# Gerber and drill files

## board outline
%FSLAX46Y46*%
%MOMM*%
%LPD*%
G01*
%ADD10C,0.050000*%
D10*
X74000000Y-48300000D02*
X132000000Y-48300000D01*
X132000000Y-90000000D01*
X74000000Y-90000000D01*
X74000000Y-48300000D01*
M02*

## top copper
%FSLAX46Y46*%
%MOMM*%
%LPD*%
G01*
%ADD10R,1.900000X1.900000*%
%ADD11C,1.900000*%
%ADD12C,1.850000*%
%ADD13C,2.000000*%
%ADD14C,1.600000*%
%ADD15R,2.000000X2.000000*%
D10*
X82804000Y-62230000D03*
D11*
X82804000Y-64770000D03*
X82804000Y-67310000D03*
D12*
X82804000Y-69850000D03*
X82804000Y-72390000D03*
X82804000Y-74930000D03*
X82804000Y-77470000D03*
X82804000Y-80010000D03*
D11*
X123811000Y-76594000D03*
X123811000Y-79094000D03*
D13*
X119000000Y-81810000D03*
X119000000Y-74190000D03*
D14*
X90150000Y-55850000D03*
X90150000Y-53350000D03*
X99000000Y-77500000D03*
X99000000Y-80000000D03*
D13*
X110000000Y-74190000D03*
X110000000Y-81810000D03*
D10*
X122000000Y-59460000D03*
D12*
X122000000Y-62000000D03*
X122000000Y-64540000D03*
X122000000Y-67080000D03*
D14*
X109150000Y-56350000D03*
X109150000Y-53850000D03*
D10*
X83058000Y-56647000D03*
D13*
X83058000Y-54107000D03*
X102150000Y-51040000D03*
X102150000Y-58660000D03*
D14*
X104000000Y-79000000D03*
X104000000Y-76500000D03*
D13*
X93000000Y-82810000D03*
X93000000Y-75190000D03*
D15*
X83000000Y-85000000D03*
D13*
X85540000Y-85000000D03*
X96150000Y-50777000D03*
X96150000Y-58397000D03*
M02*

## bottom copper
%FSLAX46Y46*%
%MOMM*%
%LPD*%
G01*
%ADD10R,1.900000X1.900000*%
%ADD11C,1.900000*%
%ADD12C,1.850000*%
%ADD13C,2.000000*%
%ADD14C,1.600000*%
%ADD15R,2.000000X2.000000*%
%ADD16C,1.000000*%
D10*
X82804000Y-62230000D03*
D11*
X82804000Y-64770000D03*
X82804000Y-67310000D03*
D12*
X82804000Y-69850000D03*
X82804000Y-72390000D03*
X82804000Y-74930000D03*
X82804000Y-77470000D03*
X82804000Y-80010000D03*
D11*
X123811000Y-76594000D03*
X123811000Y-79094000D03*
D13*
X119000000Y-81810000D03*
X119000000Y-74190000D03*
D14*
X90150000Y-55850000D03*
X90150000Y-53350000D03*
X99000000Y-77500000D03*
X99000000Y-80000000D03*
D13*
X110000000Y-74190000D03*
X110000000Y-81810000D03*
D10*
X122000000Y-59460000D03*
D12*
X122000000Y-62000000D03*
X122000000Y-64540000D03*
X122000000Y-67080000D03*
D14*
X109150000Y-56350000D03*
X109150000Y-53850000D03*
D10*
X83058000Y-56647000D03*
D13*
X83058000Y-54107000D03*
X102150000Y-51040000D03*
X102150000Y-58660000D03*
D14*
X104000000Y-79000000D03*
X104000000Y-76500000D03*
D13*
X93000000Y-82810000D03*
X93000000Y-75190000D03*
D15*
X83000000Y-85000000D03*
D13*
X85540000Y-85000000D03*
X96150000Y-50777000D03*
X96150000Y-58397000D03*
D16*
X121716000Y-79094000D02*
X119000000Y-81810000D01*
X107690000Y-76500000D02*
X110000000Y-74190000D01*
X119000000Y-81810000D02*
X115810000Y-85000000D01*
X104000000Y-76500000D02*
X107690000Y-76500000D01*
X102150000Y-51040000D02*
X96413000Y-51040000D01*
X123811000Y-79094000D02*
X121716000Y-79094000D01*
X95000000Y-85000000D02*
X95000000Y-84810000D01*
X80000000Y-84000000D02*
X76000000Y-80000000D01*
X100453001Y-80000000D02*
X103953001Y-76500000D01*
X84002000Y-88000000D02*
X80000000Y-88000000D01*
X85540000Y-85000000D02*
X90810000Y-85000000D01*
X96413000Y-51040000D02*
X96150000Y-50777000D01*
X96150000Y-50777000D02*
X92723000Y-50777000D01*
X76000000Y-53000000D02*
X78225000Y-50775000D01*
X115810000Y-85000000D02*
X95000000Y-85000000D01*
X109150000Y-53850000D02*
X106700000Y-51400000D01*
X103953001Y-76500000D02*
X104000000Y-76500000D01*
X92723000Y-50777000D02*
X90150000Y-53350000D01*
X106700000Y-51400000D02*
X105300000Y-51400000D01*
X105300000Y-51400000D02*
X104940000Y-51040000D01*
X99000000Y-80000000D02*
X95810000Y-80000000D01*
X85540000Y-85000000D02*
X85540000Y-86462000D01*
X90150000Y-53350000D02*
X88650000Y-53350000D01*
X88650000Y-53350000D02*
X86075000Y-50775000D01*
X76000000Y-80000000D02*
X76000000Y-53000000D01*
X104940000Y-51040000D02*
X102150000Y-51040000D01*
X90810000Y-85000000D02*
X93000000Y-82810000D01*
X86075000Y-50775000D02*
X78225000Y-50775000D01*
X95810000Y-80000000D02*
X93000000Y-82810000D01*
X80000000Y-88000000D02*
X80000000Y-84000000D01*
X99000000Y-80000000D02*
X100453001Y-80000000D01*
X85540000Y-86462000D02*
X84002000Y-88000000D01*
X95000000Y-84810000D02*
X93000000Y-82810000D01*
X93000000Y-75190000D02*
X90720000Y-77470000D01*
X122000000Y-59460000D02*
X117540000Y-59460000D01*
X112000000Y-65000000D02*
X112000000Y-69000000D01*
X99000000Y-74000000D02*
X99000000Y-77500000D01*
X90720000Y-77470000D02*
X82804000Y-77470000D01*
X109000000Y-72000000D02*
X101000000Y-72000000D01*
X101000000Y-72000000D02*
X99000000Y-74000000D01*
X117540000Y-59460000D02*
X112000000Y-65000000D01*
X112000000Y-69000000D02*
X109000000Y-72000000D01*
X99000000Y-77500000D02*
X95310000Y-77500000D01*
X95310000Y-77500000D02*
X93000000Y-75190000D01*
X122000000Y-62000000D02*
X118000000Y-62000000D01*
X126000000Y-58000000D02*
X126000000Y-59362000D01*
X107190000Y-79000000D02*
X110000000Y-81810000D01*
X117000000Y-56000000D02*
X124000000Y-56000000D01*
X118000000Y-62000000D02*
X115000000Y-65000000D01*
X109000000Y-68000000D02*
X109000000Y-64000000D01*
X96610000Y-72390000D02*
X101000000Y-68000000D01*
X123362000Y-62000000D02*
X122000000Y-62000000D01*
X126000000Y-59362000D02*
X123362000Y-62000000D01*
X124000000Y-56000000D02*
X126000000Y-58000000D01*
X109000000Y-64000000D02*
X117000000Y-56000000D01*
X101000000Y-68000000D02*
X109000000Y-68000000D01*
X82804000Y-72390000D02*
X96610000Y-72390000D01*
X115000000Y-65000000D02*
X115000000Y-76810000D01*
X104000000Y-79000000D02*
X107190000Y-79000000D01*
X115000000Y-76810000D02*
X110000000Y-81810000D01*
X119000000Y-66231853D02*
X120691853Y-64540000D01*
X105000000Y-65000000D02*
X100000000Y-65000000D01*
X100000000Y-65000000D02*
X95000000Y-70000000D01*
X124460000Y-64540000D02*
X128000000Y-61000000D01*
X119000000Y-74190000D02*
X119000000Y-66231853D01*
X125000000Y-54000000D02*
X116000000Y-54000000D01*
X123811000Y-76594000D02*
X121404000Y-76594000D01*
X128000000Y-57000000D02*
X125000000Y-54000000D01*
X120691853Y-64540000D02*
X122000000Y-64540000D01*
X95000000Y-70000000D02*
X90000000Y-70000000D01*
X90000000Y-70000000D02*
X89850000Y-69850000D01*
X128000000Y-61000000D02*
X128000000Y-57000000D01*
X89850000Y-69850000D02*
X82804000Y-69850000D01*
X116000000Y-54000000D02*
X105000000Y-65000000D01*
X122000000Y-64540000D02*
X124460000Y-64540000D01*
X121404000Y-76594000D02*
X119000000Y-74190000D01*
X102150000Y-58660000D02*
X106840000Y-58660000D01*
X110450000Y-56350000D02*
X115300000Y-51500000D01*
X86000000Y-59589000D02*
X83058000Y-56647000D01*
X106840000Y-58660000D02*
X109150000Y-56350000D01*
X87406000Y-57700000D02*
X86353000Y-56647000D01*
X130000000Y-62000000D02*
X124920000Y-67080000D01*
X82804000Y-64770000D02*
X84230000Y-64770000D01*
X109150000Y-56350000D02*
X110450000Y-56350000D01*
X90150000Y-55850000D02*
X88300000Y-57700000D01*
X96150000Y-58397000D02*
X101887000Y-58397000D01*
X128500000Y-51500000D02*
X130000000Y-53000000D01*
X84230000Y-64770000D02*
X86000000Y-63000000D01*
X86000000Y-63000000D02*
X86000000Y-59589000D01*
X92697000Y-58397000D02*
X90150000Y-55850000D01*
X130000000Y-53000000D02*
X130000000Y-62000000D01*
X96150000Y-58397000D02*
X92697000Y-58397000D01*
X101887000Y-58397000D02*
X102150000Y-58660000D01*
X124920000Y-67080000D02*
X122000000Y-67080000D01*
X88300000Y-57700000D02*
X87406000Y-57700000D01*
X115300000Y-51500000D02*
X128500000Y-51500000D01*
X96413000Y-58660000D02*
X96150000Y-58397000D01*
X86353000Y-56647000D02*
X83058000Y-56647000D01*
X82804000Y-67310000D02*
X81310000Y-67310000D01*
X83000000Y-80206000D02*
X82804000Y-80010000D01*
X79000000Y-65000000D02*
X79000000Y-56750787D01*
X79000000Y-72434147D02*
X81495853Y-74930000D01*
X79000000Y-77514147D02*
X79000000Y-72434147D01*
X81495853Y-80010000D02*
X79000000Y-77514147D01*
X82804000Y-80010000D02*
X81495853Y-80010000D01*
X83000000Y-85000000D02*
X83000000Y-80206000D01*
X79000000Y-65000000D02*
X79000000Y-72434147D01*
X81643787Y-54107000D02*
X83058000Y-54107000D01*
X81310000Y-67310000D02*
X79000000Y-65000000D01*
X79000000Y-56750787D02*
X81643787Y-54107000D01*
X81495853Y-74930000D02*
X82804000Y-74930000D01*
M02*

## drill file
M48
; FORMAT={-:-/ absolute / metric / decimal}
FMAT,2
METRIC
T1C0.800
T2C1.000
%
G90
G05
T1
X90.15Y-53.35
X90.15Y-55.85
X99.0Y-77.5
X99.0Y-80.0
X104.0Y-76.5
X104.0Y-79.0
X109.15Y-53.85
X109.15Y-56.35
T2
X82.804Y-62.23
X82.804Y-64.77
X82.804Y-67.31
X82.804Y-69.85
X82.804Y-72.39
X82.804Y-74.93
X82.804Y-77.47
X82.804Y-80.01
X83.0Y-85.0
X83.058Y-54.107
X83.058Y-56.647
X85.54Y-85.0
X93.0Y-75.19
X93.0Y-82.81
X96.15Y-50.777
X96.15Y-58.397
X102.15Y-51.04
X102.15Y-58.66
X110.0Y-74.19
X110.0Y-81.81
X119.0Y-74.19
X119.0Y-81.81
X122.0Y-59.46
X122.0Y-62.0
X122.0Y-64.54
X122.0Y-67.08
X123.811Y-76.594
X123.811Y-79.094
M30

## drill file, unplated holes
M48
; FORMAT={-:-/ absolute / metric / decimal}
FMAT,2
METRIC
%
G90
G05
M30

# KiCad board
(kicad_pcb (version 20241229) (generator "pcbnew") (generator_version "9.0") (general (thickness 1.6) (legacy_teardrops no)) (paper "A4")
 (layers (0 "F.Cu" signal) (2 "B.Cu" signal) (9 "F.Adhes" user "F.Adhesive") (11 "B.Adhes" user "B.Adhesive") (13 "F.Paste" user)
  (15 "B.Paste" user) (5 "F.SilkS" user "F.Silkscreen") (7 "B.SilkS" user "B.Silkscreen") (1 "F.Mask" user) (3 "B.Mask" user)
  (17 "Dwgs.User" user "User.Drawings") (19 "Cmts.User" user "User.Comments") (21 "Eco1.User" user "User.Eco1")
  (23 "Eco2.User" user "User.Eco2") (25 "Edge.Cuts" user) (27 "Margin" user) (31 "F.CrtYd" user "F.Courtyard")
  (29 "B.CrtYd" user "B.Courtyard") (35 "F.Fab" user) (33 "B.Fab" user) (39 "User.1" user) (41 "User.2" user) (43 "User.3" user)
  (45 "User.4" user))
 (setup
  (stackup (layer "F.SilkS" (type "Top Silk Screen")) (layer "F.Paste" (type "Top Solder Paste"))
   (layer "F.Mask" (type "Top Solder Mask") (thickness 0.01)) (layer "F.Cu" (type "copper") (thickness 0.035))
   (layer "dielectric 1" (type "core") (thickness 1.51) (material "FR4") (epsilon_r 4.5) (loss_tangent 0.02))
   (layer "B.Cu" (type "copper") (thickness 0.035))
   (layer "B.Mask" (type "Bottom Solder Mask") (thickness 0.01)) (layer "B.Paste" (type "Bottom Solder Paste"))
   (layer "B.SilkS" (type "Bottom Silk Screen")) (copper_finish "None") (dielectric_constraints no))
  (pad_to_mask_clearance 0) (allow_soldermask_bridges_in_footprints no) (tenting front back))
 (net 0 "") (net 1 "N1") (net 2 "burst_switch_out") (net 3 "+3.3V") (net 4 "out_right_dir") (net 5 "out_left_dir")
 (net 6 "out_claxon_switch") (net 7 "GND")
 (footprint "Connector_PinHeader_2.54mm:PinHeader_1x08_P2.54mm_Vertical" (layer "F.Cu") (at 82.804 62.23)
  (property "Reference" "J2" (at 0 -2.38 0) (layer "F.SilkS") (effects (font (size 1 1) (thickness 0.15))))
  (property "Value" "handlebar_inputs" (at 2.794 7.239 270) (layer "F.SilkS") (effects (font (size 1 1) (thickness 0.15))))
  (pad "1" thru_hole rect (at 0 0) (size 1.9 1.9) (drill 1) (layers "*.Cu" "*.Mask") (remove_unused_layers no) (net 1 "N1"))
  (pad "2" thru_hole circle (at 0 2.54) (size 1.9 1.9) (drill 1) (layers "*.Cu" "*.Mask") (remove_unused_layers no)
   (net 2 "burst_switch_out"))
  (pad "3" thru_hole circle (at 0 5.08) (size 1.9 1.9) (drill 1) (layers "*.Cu" "*.Mask") (remove_unused_layers no) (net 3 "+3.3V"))
  (pad "4" thru_hole circle (at 0 7.62) (size 1.85 1.85) (drill 1) (layers "*.Cu" "*.Mask") (remove_unused_layers no)
   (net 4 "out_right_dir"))
  (pad "5" thru_hole circle (at 0 10.16) (size 1.85 1.85) (drill 1) (layers "*.Cu" "*.Mask") (remove_unused_layers no)
   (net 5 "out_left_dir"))
  (pad "6" thru_hole circle (at 0 12.7) (size 1.85 1.85) (drill 1) (layers "*.Cu" "*.Mask") (remove_unused_layers no) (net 3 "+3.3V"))
  (pad "7" thru_hole circle (at 0 15.24) (size 1.85 1.85) (drill 1) (layers "*.Cu" "*.Mask") (remove_unused_layers no)
   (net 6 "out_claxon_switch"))
  (pad "8" thru_hole circle (at 0 17.78) (size 1.85 1.85) (drill 1) (layers "*.Cu" "*.Mask") (remove_unused_layers no) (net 3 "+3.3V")))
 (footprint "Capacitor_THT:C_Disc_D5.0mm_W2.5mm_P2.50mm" (layer "F.Cu") (at 123.811 76.594 -90)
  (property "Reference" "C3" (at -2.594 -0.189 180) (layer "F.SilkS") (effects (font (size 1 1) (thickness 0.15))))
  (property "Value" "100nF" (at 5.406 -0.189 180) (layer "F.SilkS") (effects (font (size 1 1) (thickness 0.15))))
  (pad "1" thru_hole circle (at 0 0 270) (size 1.9 1.9) (drill 1) (layers "*.Cu" "*.Mask") (remove_unused_layers no) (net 4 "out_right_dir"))
  (pad "2" thru_hole circle (at 2.5 0 270) (size 1.9 1.9) (drill 1) (layers "*.Cu" "*.Mask") (remove_unused_layers no) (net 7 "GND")))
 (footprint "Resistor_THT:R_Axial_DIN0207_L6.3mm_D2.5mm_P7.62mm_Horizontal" (layer "F.Cu") (at 119 81.81 90)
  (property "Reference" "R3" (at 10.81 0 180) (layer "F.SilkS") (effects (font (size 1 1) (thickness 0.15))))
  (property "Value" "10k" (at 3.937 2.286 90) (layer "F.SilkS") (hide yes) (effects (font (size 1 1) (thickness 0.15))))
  (pad "1" thru_hole circle (at 0 0 90) (size 2 2) (drill 1) (layers "*.Cu" "*.Mask") (remove_unused_layers no) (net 7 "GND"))
  (pad "2" thru_hole circle (at 7.62 0 90) (size 2 2) (drill 1) (layers "*.Cu" "*.Mask") (remove_unused_layers no) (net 4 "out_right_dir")))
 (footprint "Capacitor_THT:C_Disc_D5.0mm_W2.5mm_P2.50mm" (layer "F.Cu") (at 90.15 55.85 90)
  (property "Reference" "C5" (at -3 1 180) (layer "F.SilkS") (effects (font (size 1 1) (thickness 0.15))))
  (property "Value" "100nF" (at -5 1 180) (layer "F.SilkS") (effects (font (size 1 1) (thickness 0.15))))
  (pad "1" thru_hole circle (at 0 0 90) (size 1.6 1.6) (drill 0.8) (layers "*.Cu" "*.Mask") (remove_unused_layers no)
   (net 2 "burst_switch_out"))
  (pad "2" thru_hole circle (at 2.5 0 90) (size 1.6 1.6) (drill 0.8) (layers "*.Cu" "*.Mask") (remove_unused_layers no) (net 7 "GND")))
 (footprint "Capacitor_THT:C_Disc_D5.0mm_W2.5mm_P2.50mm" (layer "F.Cu") (at 99 77.5 -90)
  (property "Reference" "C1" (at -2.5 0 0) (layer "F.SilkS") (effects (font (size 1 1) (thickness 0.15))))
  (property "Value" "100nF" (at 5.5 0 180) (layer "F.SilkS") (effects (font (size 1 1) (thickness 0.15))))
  (pad "1" thru_hole circle (at 0 0 270) (size 1.6 1.6) (drill 0.8) (layers "*.Cu" "*.Mask") (remove_unused_layers no)
   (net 6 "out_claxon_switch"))
  (pad "2" thru_hole circle (at 2.5 0 270) (size 1.6 1.6) (drill 0.8) (layers "*.Cu" "*.Mask") (remove_unused_layers no) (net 7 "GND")))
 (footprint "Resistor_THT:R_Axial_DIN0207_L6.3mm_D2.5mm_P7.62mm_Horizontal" (layer "F.Cu") (at 110 74.19 -90)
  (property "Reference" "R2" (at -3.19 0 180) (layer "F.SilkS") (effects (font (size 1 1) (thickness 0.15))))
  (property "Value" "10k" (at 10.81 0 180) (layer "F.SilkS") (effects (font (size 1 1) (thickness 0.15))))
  (pad "1" thru_hole circle (at 0 0 270) (size 2 2) (drill 1) (layers "*.Cu" "*.Mask") (remove_unused_layers no) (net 7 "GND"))
  (pad "2" thru_hole circle (at 7.62 0 270) (size 2 2) (drill 1) (layers "*.Cu" "*.Mask") (remove_unused_layers no) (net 5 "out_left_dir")))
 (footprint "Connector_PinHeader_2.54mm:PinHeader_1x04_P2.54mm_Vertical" (layer "F.Cu") (at 122 59.46)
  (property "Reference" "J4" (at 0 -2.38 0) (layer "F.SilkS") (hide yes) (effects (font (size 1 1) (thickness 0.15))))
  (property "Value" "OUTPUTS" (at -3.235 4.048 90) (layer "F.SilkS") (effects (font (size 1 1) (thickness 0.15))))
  (pad "1" thru_hole rect (at 0 0) (size 1.9 1.9) (drill 1) (layers "*.Cu" "*.Mask") (remove_unused_layers no) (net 6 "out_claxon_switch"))
  (pad "2" thru_hole circle (at 0 2.54) (size 1.85 1.85) (drill 1) (layers "*.Cu" "*.Mask") (remove_unused_layers no) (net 5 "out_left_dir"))
  (pad "3" thru_hole circle (at 0 5.08) (size 1.85 1.85) (drill 1) (layers "*.Cu" "*.Mask") (remove_unused_layers no)
   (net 4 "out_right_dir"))
  (pad "4" thru_hole circle (at 0 7.62) (size 1.85 1.85) (drill 1) (layers "*.Cu" "*.Mask") (remove_unused_layers no)
   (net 2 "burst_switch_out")))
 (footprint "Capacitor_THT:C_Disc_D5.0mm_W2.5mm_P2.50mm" (layer "F.Cu") (at 109.15 56.35 90)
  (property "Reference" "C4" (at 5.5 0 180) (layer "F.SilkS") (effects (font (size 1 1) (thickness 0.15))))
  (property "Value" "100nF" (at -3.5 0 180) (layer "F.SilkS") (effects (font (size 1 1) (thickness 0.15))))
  (pad "1" thru_hole circle (at 0 0 90) (size 1.6 1.6) (drill 0.8) (layers "*.Cu" "*.Mask") (remove_unused_layers no)
   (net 2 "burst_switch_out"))
  (pad "2" thru_hole circle (at 2.5 0 90.798) (size 1.6 1.6) (drill 0.8) (layers "*.Cu" "*.Mask") (remove_unused_layers no) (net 7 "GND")))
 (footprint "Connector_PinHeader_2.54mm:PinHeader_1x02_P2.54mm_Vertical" (layer "F.Cu") (at 83.058 56.647 180)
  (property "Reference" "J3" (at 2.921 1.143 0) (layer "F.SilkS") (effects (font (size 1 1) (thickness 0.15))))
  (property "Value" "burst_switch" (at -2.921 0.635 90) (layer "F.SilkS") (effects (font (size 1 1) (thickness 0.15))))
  (pad "1" thru_hole rect (at 0 0 180) (size 1.9 1.9) (drill 1) (layers "*.Cu" "*.Mask") (remove_unused_layers no)
   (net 2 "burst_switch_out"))
  (pad "2" thru_hole circle (at 0 2.54 180) (size 2 2) (drill 1) (layers "*.Cu" "*.Mask") (remove_unused_layers no) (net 3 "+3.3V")))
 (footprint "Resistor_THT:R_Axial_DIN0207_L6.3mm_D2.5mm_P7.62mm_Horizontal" (layer "F.Cu") (at 102.15 51.04 -90)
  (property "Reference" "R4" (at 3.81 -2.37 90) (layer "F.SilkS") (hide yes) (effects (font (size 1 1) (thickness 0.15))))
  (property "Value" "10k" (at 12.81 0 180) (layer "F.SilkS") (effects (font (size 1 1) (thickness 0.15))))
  (pad "1" thru_hole circle (at 0 0 270) (size 2 2) (drill 1) (layers "*.Cu" "*.Mask") (remove_unused_layers no) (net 7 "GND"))
  (pad "2" thru_hole circle (at 7.62 0 270) (size 2 2) (drill 1) (layers "*.Cu" "*.Mask") (remove_unused_layers no)
   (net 2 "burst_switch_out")))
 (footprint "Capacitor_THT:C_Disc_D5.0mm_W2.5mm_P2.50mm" (layer "F.Cu") (at 104 79 90)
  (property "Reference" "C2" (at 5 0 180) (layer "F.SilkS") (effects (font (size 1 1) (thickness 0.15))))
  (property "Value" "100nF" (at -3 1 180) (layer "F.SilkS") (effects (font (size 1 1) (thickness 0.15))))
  (pad "1" thru_hole circle (at 0 0 90) (size 1.6 1.6) (drill 0.8) (layers "*.Cu" "*.Mask") (remove_unused_layers no) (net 5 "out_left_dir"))
  (pad "2" thru_hole circle (at 2.5 0 90) (size 1.6 1.6) (drill 0.8) (layers "*.Cu" "*.Mask") (remove_unused_layers no) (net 7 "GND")))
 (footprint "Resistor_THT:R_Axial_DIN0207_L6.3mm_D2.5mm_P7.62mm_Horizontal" (layer "F.Cu") (at 93 82.81 90)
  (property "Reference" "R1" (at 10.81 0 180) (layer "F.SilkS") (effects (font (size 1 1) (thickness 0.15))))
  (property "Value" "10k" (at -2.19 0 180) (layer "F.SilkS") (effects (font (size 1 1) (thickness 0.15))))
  (pad "1" thru_hole circle (at 0 0 90) (size 2 2) (drill 1) (layers "*.Cu" "*.Mask") (remove_unused_layers no) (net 7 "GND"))
  (pad "2" thru_hole circle (at 7.62 0 90) (size 2 2) (drill 1) (layers "*.Cu" "*.Mask") (remove_unused_layers no)
   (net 6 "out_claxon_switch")))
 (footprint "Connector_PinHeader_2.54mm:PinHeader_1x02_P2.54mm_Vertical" (layer "F.Cu") (at 83 85 90)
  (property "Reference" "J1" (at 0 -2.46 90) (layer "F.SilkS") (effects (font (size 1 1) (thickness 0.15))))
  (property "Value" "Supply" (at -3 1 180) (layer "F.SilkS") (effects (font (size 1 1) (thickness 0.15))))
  (pad "1" thru_hole rect (at 0 0 90) (size 2 2) (drill 1) (layers "*.Cu" "*.Mask") (remove_unused_layers no) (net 3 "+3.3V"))
  (pad "2" thru_hole circle (at 0 2.54 90) (size 2 2) (drill 1) (layers "*.Cu" "*.Mask") (remove_unused_layers no) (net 7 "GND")))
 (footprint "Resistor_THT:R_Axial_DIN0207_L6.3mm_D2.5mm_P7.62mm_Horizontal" (layer "F.Cu") (at 96.15 50.777 -90)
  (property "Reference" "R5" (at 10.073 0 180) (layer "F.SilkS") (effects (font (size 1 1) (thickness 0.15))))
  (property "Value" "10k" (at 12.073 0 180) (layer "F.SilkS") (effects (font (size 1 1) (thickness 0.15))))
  (pad "1" thru_hole circle (at 0 0 270) (size 2 2) (drill 1) (layers "*.Cu" "*.Mask") (remove_unused_layers no) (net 7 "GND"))
  (pad "2" thru_hole circle (at 7.62 0 270) (size 2 2) (drill 1) (layers "*.Cu" "*.Mask") (remove_unused_layers no)
   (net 2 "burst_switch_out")))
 (gr_rect (start 74 48.3) (end 132 90) (stroke (width 0.05) (type default)) (fill no) (layer "Edge.Cuts"))
 (segment (start 121.716 79.094) (end 119 81.81) (width 1) (layer "B.Cu") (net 7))
 (segment (start 107.69 76.5) (end 110 74.19) (width 1) (layer "B.Cu") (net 7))
 (segment (start 119 81.81) (end 115.81 85) (width 1) (layer "B.Cu") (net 7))
 (segment (start 104 76.5) (end 107.69 76.5) (width 1) (layer "B.Cu") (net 7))
 (segment (start 102.15 51.04) (end 96.413 51.04) (width 1) (layer "B.Cu") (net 7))
 (segment (start 123.811 79.094) (end 121.716 79.094) (width 1) (layer "B.Cu") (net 7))
 (segment (start 95 85) (end 95 84.81) (width 1) (layer "B.Cu") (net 7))
 (segment (start 80 84) (end 76 80) (width 1) (layer "B.Cu") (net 7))
 (segment (start 100.453001 80) (end 103.953001 76.5) (width 1) (layer "B.Cu") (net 7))
 (segment (start 84.002 88) (end 80 88) (width 1) (layer "B.Cu") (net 7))
 (segment (start 85.54 85) (end 90.81 85) (width 1) (layer "B.Cu") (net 7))
 (segment (start 96.413 51.04) (end 96.15 50.777) (width 1) (layer "B.Cu") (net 7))
 (segment (start 96.15 50.777) (end 92.723 50.777) (width 1) (layer "B.Cu") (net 7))
 (segment (start 76 53) (end 78.225 50.775) (width 1) (layer "B.Cu") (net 7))
 (segment (start 115.81 85) (end 95 85) (width 1) (layer "B.Cu") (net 7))
 (segment (start 109.15 53.85) (end 106.7 51.4) (width 1) (layer "B.Cu") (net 7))
 (segment (start 103.953001 76.5) (end 104 76.5) (width 1) (layer "B.Cu") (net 7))
 (segment (start 92.723 50.777) (end 90.15 53.35) (width 1) (layer "B.Cu") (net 7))
 (segment (start 106.7 51.4) (end 105.3 51.4) (width 1) (layer "B.Cu") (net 7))
 (segment (start 105.3 51.4) (end 104.94 51.04) (width 1) (layer "B.Cu") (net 7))
 (segment (start 99 80) (end 95.81 80) (width 1) (layer "B.Cu") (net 7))
 (segment (start 85.54 85) (end 85.54 86.462) (width 1) (layer "B.Cu") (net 7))
 (segment (start 90.15 53.35) (end 88.65 53.35) (width 1) (layer "B.Cu") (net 7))
 (segment (start 88.65 53.35) (end 86.075 50.775) (width 1) (layer "B.Cu") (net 7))
 (segment (start 76 80) (end 76 53) (width 1) (layer "B.Cu") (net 7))
 (segment (start 104.94 51.04) (end 102.15 51.04) (width 1) (layer "B.Cu") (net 7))
 (segment (start 90.81 85) (end 93 82.81) (width 1) (layer "B.Cu") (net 7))
 (segment (start 86.075 50.775) (end 78.225 50.775) (width 1) (layer "B.Cu") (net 7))
 (segment (start 95.81 80) (end 93 82.81) (width 1) (layer "B.Cu") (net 7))
 (segment (start 80 88) (end 80 84) (width 1) (layer "B.Cu") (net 7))
 (segment (start 99 80) (end 100.453001 80) (width 1) (layer "B.Cu") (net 7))
 (segment (start 85.54 86.462) (end 84.002 88) (width 1) (layer "B.Cu") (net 7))
 (segment (start 95 84.81) (end 93 82.81) (width 1) (layer "B.Cu") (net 7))
 (segment (start 93 75.19) (end 90.72 77.47) (width 1) (layer "B.Cu") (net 6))
 (segment (start 122 59.46) (end 117.54 59.46) (width 1) (layer "B.Cu") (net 6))
 (segment (start 112 65) (end 112 69) (width 1) (layer "B.Cu") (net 6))
 (segment (start 99 74) (end 99 77.5) (width 1) (layer "B.Cu") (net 6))
 (segment (start 90.72 77.47) (end 82.804 77.47) (width 1) (layer "B.Cu") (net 6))
 (segment (start 109 72) (end 101 72) (width 1) (layer "B.Cu") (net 6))
 (segment (start 101 72) (end 99 74) (width 1) (layer "B.Cu") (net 6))
 (segment (start 117.54 59.46) (end 112 65) (width 1) (layer "B.Cu") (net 6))
 (segment (start 112 69) (end 109 72) (width 1) (layer "B.Cu") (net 6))
 (segment (start 99 77.5) (end 95.31 77.5) (width 1) (layer "B.Cu") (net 6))
 (segment (start 95.31 77.5) (end 93 75.19) (width 1) (layer "B.Cu") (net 6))
 (segment (start 122 62) (end 118 62) (width 1) (layer "B.Cu") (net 5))
 (segment (start 126 58) (end 126 59.362) (width 1) (layer "B.Cu") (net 5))
 (segment (start 107.19 79) (end 110 81.81) (width 1) (layer "B.Cu") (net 5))
 (segment (start 117 56) (end 124 56) (width 1) (layer "B.Cu") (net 5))
 (segment (start 118 62) (end 115 65) (width 1) (layer "B.Cu") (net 5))
 (segment (start 109 68) (end 109 64) (width 1) (layer "B.Cu") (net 5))
 (segment (start 96.61 72.39) (end 101 68) (width 1) (layer "B.Cu") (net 5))
 (segment (start 123.362 62) (end 122 62) (width 1) (layer "B.Cu") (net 5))
 (segment (start 126 59.362) (end 123.362 62) (width 1) (layer "B.Cu") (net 5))
 (segment (start 124 56) (end 126 58) (width 1) (layer "B.Cu") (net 5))
 (segment (start 109 64) (end 117 56) (width 1) (layer "B.Cu") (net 5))
 (segment (start 101 68) (end 109 68) (width 1) (layer "B.Cu") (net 5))
 (segment (start 82.804 72.39) (end 96.61 72.39) (width 1) (layer "B.Cu") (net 5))
 (segment (start 115 65) (end 115 76.81) (width 1) (layer "B.Cu") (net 5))
 (segment (start 104 79) (end 107.19 79) (width 1) (layer "B.Cu") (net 5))
 (segment (start 115 76.81) (end 110 81.81) (width 1) (layer "B.Cu") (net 5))
 (segment (start 119 66.231853) (end 120.691853 64.54) (width 1) (layer "B.Cu") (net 4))
 (segment (start 105 65) (end 100 65) (width 1) (layer "B.Cu") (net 4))
 (segment (start 100 65) (end 95 70) (width 1) (layer "B.Cu") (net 4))
 (segment (start 124.46 64.54) (end 128 61) (width 1) (layer "B.Cu") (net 4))
 (segment (start 119 74.19) (end 119 66.231853) (width 1) (layer "B.Cu") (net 4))
 (segment (start 125 54) (end 116 54) (width 1) (layer "B.Cu") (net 4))
 (segment (start 123.811 76.594) (end 121.404 76.594) (width 1) (layer "B.Cu") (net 4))
 (segment (start 128 57) (end 125 54) (width 1) (layer "B.Cu") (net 4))
 (segment (start 120.691853 64.54) (end 122 64.54) (width 1) (layer "B.Cu") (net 4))
 (segment (start 95 70) (end 90 70) (width 1) (layer "B.Cu") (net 4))
 (segment (start 90 70) (end 89.85 69.85) (width 1) (layer "B.Cu") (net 4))
 (segment (start 128 61) (end 128 57) (width 1) (layer "B.Cu") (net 4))
 (segment (start 89.85 69.85) (end 82.804 69.85) (width 1) (layer "B.Cu") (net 4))
 (segment (start 116 54) (end 105 65) (width 1) (layer "B.Cu") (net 4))
 (segment (start 122 64.54) (end 124.46 64.54) (width 1) (layer "B.Cu") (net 4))
 (segment (start 121.404 76.594) (end 119 74.19) (width 1) (layer "B.Cu") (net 4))
 (segment (start 102.15 58.66) (end 106.84 58.66) (width 1) (layer "B.Cu") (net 2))
 (segment (start 110.45 56.35) (end 115.3 51.5) (width 1) (layer "B.Cu") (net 2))
 (segment (start 86 59.589) (end 83.058 56.647) (width 1) (layer "B.Cu") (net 2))
 (segment (start 106.84 58.66) (end 109.15 56.35) (width 1) (layer "B.Cu") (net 2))
 (segment (start 87.406 57.7) (end 86.353 56.647) (width 1) (layer "B.Cu") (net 2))
 (segment (start 130 62) (end 124.92 67.08) (width 1) (layer "B.Cu") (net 2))
 (segment (start 82.804 64.77) (end 84.23 64.77) (width 1) (layer "B.Cu") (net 2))
 (segment (start 109.15 56.35) (end 110.45 56.35) (width 1) (layer "B.Cu") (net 2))
 (segment (start 90.15 55.85) (end 88.3 57.7) (width 1) (layer "B.Cu") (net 2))
 (segment (start 96.15 58.397) (end 101.887 58.397) (width 1) (layer "B.Cu") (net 2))
 (segment (start 128.5 51.5) (end 130 53) (width 1) (layer "B.Cu") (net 2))
 (segment (start 84.23 64.77) (end 86 63) (width 1) (layer "B.Cu") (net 2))
 (segment (start 86 63) (end 86 59.589) (width 1) (layer "B.Cu") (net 2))
 (segment (start 92.697 58.397) (end 90.15 55.85) (width 1) (layer "B.Cu") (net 2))
 (segment (start 130 53) (end 130 62) (width 1) (layer "B.Cu") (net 2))
 (segment (start 96.15 58.397) (end 92.697 58.397) (width 1) (layer "B.Cu") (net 2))
 (segment (start 101.887 58.397) (end 102.15 58.66) (width 1) (layer "B.Cu") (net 2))
 (segment (start 124.92 67.08) (end 122 67.08) (width 1) (layer "B.Cu") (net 2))
 (segment (start 88.3 57.7) (end 87.406 57.7) (width 1) (layer "B.Cu") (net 2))
 (segment (start 115.3 51.5) (end 128.5 51.5) (width 1) (layer "B.Cu") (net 2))
 (segment (start 96.413 58.66) (end 96.15 58.397) (width 1) (layer "B.Cu") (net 2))
 (segment (start 86.353 56.647) (end 83.058 56.647) (width 1) (layer "B.Cu") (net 2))
 (segment (start 82.804 67.31) (end 81.31 67.31) (width 1) (layer "B.Cu") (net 3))
 (segment (start 83 80.206) (end 82.804 80.01) (width 1) (layer "B.Cu") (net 3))
 (segment (start 79 65) (end 79 56.750787) (width 1) (layer "B.Cu") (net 3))
 (segment (start 79 72.434147) (end 81.495853 74.93) (width 1) (layer "B.Cu") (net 3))
 (segment (start 79 77.514147) (end 79 72.434147) (width 1) (layer "B.Cu") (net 3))
 (segment (start 81.495853 80.01) (end 79 77.514147) (width 1) (layer "B.Cu") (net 3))
 (segment (start 82.804 80.01) (end 81.495853 80.01) (width 1) (layer "B.Cu") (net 3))
 (segment (start 83 85) (end 83 80.206) (width 1) (layer "B.Cu") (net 3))
 (segment (start 79 65) (end 79 72.434147) (width 1) (layer "B.Cu") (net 3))
 (segment (start 81.643787 54.107) (end 83.058 54.107) (width 1) (layer "B.Cu") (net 3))
 (segment (start 81.31 67.31) (end 79 65) (width 1) (layer "B.Cu") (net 3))
 (segment (start 79 56.750787) (end 81.643787 54.107) (width 1) (layer "B.Cu") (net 3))
 (segment (start 81.495853 74.93) (end 82.804 74.93) (width 1) (layer "B.Cu") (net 3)))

